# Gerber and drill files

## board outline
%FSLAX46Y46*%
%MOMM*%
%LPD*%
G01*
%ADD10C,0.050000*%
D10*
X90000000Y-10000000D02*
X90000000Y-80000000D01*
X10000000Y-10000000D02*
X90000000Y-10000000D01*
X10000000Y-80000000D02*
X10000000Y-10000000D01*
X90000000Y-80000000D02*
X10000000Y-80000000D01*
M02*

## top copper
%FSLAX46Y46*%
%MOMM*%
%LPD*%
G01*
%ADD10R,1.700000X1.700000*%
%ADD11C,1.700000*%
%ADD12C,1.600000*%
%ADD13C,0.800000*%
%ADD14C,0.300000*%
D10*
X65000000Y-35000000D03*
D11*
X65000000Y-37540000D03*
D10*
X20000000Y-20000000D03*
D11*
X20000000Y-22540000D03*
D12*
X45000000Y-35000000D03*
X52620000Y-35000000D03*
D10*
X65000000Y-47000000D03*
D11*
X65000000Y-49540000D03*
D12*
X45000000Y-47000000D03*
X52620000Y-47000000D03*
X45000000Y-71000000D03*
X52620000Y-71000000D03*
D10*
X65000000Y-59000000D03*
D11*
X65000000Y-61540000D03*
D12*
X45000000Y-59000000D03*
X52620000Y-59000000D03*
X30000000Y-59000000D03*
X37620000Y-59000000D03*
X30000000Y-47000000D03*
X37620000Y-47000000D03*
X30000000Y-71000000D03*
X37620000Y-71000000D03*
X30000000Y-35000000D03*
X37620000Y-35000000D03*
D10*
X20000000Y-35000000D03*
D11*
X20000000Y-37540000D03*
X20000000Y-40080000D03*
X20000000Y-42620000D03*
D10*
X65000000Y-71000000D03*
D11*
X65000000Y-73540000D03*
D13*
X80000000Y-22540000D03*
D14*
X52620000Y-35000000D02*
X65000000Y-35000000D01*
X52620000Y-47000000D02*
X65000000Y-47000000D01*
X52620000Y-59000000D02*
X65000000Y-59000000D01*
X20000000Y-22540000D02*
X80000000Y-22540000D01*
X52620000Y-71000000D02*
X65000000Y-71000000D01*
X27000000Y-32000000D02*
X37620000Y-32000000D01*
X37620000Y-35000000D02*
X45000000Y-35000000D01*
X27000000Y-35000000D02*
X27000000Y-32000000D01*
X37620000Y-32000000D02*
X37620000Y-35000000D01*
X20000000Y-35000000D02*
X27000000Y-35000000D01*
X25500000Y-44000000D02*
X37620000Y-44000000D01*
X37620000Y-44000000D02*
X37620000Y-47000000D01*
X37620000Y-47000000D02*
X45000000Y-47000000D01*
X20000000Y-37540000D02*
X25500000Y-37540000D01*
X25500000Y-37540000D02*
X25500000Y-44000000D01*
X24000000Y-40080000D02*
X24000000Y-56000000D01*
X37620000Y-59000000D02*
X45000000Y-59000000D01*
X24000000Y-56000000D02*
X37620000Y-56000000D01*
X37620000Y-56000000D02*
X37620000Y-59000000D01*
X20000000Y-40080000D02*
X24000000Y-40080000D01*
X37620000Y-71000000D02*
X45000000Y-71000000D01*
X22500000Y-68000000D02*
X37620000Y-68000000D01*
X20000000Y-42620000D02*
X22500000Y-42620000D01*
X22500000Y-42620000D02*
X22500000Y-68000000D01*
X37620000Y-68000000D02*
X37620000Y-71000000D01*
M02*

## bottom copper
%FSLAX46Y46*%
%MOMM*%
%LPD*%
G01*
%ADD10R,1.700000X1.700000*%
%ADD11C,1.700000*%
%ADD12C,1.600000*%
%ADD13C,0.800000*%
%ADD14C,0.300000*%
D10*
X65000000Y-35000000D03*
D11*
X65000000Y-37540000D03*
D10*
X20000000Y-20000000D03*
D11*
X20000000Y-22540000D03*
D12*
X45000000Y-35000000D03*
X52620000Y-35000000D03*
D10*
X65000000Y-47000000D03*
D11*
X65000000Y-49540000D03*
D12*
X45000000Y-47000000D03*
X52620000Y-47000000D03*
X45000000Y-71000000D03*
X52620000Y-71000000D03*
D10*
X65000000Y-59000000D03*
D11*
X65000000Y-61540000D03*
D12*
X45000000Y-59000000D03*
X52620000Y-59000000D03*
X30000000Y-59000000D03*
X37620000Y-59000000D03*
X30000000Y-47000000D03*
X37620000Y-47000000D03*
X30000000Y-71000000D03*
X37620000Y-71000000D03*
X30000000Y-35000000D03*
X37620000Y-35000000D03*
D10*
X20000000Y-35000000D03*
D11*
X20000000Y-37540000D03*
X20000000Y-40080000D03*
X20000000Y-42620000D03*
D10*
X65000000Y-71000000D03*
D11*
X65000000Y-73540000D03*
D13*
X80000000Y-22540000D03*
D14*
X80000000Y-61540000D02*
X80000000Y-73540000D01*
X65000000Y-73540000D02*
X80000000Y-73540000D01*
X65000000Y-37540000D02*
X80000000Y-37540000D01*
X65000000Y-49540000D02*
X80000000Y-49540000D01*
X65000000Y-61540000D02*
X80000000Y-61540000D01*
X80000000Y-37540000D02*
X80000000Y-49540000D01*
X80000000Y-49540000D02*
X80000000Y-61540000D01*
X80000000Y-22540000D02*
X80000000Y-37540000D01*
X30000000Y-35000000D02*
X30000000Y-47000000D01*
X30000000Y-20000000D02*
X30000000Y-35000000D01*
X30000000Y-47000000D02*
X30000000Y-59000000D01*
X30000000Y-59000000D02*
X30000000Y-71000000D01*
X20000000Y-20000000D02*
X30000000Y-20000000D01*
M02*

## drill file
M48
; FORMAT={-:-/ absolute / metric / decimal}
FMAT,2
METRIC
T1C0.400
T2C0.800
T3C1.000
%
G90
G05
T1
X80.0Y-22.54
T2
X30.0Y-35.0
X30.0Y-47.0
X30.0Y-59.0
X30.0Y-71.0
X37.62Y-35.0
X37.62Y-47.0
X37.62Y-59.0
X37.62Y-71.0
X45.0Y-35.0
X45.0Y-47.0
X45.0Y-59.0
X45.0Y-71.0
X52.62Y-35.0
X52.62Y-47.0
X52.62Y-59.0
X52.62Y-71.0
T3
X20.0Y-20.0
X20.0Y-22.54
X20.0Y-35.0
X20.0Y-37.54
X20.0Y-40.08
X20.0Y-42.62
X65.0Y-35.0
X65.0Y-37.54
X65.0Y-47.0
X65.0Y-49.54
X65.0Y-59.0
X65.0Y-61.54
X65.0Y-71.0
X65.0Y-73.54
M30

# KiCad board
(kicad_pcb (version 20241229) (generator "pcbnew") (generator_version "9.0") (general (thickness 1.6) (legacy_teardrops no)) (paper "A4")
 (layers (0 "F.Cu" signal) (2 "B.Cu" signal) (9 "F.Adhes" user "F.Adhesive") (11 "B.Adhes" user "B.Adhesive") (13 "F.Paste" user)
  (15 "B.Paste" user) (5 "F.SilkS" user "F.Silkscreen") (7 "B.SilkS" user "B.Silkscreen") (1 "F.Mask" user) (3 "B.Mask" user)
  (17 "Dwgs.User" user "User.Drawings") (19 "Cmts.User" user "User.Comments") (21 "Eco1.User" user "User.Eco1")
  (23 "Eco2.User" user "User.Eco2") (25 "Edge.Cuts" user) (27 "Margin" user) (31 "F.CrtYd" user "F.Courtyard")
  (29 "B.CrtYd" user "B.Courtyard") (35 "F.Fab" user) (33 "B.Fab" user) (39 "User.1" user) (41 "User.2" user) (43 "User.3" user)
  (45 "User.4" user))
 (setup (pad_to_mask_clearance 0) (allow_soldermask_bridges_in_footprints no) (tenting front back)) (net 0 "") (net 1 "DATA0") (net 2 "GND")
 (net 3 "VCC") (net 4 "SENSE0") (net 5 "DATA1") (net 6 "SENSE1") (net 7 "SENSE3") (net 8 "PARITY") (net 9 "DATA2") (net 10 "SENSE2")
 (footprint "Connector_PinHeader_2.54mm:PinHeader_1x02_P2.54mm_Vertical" (layer "F.Cu") (at 65 35)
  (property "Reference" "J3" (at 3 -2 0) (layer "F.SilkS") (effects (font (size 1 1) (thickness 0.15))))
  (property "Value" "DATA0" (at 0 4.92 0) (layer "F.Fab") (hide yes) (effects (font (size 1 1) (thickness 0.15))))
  (pad "1" thru_hole rect (at 0 0) (size 1.7 1.7) (drill 1) (layers "*.Cu" "*.Mask") (remove_unused_layers no) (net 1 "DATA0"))
  (pad "2" thru_hole circle (at 0 2.54) (size 1.7 1.7) (drill 1) (layers "*.Cu" "*.Mask") (remove_unused_layers no) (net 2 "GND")))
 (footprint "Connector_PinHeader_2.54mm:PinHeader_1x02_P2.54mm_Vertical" (layer "F.Cu") (at 20 20)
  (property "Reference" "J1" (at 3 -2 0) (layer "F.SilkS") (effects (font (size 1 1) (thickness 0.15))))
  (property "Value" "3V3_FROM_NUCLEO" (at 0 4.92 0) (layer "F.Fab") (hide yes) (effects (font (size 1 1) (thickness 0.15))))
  (pad "1" thru_hole rect (at 0 0) (size 1.7 1.7) (drill 1) (layers "*.Cu" "*.Mask") (remove_unused_layers no) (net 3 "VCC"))
  (pad "2" thru_hole circle (at 0 2.54) (size 1.7 1.7) (drill 1) (layers "*.Cu" "*.Mask") (remove_unused_layers no) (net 2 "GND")))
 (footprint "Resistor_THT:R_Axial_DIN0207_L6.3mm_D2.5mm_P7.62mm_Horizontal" (layer "F.Cu") (at 45 35)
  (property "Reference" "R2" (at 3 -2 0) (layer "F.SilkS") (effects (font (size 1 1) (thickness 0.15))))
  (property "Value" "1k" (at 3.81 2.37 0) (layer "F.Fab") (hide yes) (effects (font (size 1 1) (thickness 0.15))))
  (pad "1" thru_hole circle (at 0 0) (size 1.6 1.6) (drill 0.8) (layers "*.Cu" "*.Mask") (remove_unused_layers no) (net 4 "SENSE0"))
  (pad "2" thru_hole circle (at 7.62 0) (size 1.6 1.6) (drill 0.8) (layers "*.Cu" "*.Mask") (remove_unused_layers no) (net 1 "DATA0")))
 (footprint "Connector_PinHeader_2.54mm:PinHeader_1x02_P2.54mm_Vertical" (layer "F.Cu") (at 65 47)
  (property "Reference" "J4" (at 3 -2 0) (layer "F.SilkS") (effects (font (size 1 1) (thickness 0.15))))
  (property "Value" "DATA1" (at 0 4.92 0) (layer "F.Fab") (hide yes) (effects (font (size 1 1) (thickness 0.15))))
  (pad "1" thru_hole rect (at 0 0) (size 1.7 1.7) (drill 1) (layers "*.Cu" "*.Mask") (remove_unused_layers no) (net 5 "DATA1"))
  (pad "2" thru_hole circle (at 0 2.54) (size 1.7 1.7) (drill 1) (layers "*.Cu" "*.Mask") (remove_unused_layers no) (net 2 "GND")))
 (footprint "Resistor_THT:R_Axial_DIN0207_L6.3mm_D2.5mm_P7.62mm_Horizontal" (layer "F.Cu") (at 45 47)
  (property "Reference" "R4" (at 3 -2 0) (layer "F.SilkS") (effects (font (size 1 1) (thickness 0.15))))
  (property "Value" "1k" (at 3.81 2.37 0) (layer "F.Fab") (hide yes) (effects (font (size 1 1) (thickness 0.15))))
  (pad "1" thru_hole circle (at 0 0) (size 1.6 1.6) (drill 0.8) (layers "*.Cu" "*.Mask") (remove_unused_layers no) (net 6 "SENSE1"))
  (pad "2" thru_hole circle (at 7.62 0) (size 1.6 1.6) (drill 0.8) (layers "*.Cu" "*.Mask") (remove_unused_layers no) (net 5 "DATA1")))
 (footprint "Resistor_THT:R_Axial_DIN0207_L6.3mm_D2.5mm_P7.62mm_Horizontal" (layer "F.Cu") (at 45 71)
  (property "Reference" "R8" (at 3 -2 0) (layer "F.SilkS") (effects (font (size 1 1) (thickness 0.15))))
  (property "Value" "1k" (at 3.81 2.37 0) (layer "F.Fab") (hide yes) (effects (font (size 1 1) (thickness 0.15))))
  (pad "1" thru_hole circle (at 0 0) (size 1.6 1.6) (drill 0.8) (layers "*.Cu" "*.Mask") (remove_unused_layers no) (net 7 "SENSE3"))
  (pad "2" thru_hole circle (at 7.62 0) (size 1.6 1.6) (drill 0.8) (layers "*.Cu" "*.Mask") (remove_unused_layers no) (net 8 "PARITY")))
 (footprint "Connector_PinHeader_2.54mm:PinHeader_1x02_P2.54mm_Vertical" (layer "F.Cu") (at 65 59)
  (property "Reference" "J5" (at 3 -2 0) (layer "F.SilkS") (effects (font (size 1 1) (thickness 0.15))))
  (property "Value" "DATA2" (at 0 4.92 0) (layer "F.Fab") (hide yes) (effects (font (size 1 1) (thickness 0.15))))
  (pad "1" thru_hole rect (at 0 0) (size 1.7 1.7) (drill 1) (layers "*.Cu" "*.Mask") (remove_unused_layers no) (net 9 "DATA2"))
  (pad "2" thru_hole circle (at 0 2.54) (size 1.7 1.7) (drill 1) (layers "*.Cu" "*.Mask") (remove_unused_layers no) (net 2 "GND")))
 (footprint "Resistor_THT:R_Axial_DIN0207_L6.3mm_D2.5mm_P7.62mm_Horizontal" (layer "F.Cu") (at 45 59)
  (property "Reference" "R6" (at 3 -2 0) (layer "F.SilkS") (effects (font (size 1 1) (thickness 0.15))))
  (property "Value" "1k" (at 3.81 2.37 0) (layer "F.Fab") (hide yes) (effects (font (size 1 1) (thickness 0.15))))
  (pad "1" thru_hole circle (at 0 0) (size 1.6 1.6) (drill 0.8) (layers "*.Cu" "*.Mask") (remove_unused_layers no) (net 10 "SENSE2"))
  (pad "2" thru_hole circle (at 7.62 0) (size 1.6 1.6) (drill 0.8) (layers "*.Cu" "*.Mask") (remove_unused_layers no) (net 9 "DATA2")))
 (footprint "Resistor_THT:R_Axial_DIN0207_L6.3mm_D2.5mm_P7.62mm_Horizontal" (layer "F.Cu") (at 30 59)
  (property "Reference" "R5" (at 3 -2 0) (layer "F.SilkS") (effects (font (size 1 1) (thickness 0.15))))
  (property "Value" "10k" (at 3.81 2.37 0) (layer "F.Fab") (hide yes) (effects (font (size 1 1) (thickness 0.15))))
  (pad "1" thru_hole circle (at 0 0) (size 1.6 1.6) (drill 0.8) (layers "*.Cu" "*.Mask") (remove_unused_layers no) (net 3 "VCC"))
  (pad "2" thru_hole circle (at 7.62 0) (size 1.6 1.6) (drill 0.8) (layers "*.Cu" "*.Mask") (remove_unused_layers no) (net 10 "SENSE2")))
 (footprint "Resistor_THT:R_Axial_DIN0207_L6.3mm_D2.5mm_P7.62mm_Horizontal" (layer "F.Cu") (at 30 47)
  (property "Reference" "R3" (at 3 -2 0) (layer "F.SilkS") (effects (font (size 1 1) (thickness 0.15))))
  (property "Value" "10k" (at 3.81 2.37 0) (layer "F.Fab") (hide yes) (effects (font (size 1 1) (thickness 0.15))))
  (pad "1" thru_hole circle (at 0 0) (size 1.6 1.6) (drill 0.8) (layers "*.Cu" "*.Mask") (remove_unused_layers no) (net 3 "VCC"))
  (pad "2" thru_hole circle (at 7.62 0) (size 1.6 1.6) (drill 0.8) (layers "*.Cu" "*.Mask") (remove_unused_layers no) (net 6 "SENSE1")))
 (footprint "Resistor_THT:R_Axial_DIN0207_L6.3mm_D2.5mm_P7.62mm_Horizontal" (layer "F.Cu") (at 30 71)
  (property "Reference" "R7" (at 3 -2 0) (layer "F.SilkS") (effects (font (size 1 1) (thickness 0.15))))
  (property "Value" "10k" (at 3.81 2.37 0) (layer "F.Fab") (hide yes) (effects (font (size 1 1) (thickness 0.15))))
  (pad "1" thru_hole circle (at 0 0) (size 1.6 1.6) (drill 0.8) (layers "*.Cu" "*.Mask") (remove_unused_layers no) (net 3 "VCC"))
  (pad "2" thru_hole circle (at 7.62 0) (size 1.6 1.6) (drill 0.8) (layers "*.Cu" "*.Mask") (remove_unused_layers no) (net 7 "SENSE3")))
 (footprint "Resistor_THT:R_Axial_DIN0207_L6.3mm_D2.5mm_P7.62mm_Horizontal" (layer "F.Cu") (at 30 35)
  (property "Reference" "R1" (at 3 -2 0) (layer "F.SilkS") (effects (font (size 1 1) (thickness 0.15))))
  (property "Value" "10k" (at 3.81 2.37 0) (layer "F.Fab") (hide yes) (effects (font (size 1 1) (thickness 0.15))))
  (pad "1" thru_hole circle (at 0 0) (size 1.6 1.6) (drill 0.8) (layers "*.Cu" "*.Mask") (remove_unused_layers no) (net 3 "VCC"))
  (pad "2" thru_hole circle (at 7.62 0) (size 1.6 1.6) (drill 0.8) (layers "*.Cu" "*.Mask") (remove_unused_layers no) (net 4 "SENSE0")))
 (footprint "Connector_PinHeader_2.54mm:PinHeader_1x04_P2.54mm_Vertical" (layer "F.Cu") (at 20 35)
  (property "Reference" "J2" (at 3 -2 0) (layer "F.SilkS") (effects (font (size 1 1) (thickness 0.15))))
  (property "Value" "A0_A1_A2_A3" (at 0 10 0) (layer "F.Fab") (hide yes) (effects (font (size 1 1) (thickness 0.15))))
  (pad "1" thru_hole rect (at 0 0) (size 1.7 1.7) (drill 1) (layers "*.Cu" "*.Mask") (remove_unused_layers no) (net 4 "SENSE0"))
  (pad "2" thru_hole circle (at 0 2.54) (size 1.7 1.7) (drill 1) (layers "*.Cu" "*.Mask") (remove_unused_layers no) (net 6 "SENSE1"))
  (pad "3" thru_hole circle (at 0 5.08) (size 1.7 1.7) (drill 1) (layers "*.Cu" "*.Mask") (remove_unused_layers no) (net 10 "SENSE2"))
  (pad "4" thru_hole circle (at 0 7.62) (size 1.7 1.7) (drill 1) (layers "*.Cu" "*.Mask") (remove_unused_layers no) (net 7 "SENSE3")))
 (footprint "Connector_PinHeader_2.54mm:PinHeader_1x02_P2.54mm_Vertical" (layer "F.Cu") (at 65 71)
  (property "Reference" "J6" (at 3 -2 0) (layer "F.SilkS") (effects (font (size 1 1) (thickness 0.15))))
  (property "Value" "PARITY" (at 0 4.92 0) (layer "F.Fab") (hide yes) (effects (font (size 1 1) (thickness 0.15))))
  (pad "1" thru_hole rect (at 0 0) (size 1.7 1.7) (drill 1) (layers "*.Cu" "*.Mask") (remove_unused_layers no) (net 8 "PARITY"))
  (pad "2" thru_hole circle (at 0 2.54) (size 1.7 1.7) (drill 1) (layers "*.Cu" "*.Mask") (remove_unused_layers no) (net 2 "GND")))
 (gr_line (start 90 10) (end 90 80) (stroke (width 0.05) (type default)) (layer "Edge.Cuts"))
 (gr_line (start 10 10) (end 90 10) (stroke (width 0.05) (type default)) (layer "Edge.Cuts"))
 (gr_line (start 10 80) (end 10 10) (stroke (width 0.05) (type default)) (layer "Edge.Cuts"))
 (gr_line (start 90 80) (end 10 80) (stroke (width 0.05) (type default)) (layer "Edge.Cuts"))
 (segment (start 52.62 35) (end 65 35) (width 0.3) (layer "F.Cu") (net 1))
 (segment (start 52.62 47) (end 65 47) (width 0.3) (layer "F.Cu") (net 5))
 (segment (start 52.62 59) (end 65 59) (width 0.3) (layer "F.Cu") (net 9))
 (segment (start 20 22.54) (end 80 22.54) (width 0.3) (layer "F.Cu") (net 2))
 (via (at 80 22.54) (size 0.8) (drill 0.4) (layers "F.Cu" "B.Cu") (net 2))
 (segment (start 80 61.54) (end 80 73.54) (width 0.3) (layer "B.Cu") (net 2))
 (segment (start 65 73.54) (end 80 73.54) (width 0.3) (layer "B.Cu") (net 2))
 (segment (start 65 37.54) (end 80 37.54) (width 0.3) (layer "B.Cu") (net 2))
 (segment (start 65 49.54) (end 80 49.54) (width 0.3) (layer "B.Cu") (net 2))
 (segment (start 65 61.54) (end 80 61.54) (width 0.3) (layer "B.Cu") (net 2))
 (segment (start 80 37.54) (end 80 49.54) (width 0.3) (layer "B.Cu") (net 2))
 (segment (start 80 49.54) (end 80 61.54) (width 0.3) (layer "B.Cu") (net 2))
 (segment (start 80 22.54) (end 80 37.54) (width 0.3) (layer "B.Cu") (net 2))
 (segment (start 52.62 71) (end 65 71) (width 0.3) (layer "F.Cu") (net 8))
 (segment (start 27 32) (end 37.62 32) (width 0.3) (layer "F.Cu") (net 4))
 (segment (start 37.62 35) (end 45 35) (width 0.3) (layer "F.Cu") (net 4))
 (segment (start 27 35) (end 27 32) (width 0.3) (layer "F.Cu") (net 4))
 (segment (start 37.62 32) (end 37.62 35) (width 0.3) (layer "F.Cu") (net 4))
 (segment (start 20 35) (end 27 35) (width 0.3) (layer "F.Cu") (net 4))
 (segment (start 25.5 44) (end 37.62 44) (width 0.3) (layer "F.Cu") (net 6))
 (segment (start 37.62 44) (end 37.62 47) (width 0.3) (layer "F.Cu") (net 6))
 (segment (start 37.62 47) (end 45 47) (width 0.3) (layer "F.Cu") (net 6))
 (segment (start 20 37.54) (end 25.5 37.54) (width 0.3) (layer "F.Cu") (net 6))
 (segment (start 25.5 37.54) (end 25.5 44) (width 0.3) (layer "F.Cu") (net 6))
 (segment (start 24 40.08) (end 24 56) (width 0.3) (layer "F.Cu") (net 10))
 (segment (start 37.62 59) (end 45 59) (width 0.3) (layer "F.Cu") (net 10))
 (segment (start 24 56) (end 37.62 56) (width 0.3) (layer "F.Cu") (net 10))
 (segment (start 37.62 56) (end 37.62 59) (width 0.3) (layer "F.Cu") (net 10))
 (segment (start 20 40.08) (end 24 40.08) (width 0.3) (layer "F.Cu") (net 10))
 (segment (start 37.62 71) (end 45 71) (width 0.3) (layer "F.Cu") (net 7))
 (segment (start 22.5 68) (end 37.62 68) (width 0.3) (layer "F.Cu") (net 7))
 (segment (start 20 42.62) (end 22.5 42.62) (width 0.3) (layer "F.Cu") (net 7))
 (segment (start 22.5 42.62) (end 22.5 68) (width 0.3) (layer "F.Cu") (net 7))
 (segment (start 37.62 68) (end 37.62 71) (width 0.3) (layer "F.Cu") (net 7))
 (segment (start 30 35) (end 30 47) (width 0.3) (layer "B.Cu") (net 3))
 (segment (start 30 20) (end 30 35) (width 0.3) (layer "B.Cu") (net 3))
 (segment (start 30 47) (end 30 59) (width 0.3) (layer "B.Cu") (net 3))
 (segment (start 30 59) (end 30 71) (width 0.3) (layer "B.Cu") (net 3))
 (segment (start 20 20) (end 30 20) (width 0.3) (layer "B.Cu") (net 3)))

